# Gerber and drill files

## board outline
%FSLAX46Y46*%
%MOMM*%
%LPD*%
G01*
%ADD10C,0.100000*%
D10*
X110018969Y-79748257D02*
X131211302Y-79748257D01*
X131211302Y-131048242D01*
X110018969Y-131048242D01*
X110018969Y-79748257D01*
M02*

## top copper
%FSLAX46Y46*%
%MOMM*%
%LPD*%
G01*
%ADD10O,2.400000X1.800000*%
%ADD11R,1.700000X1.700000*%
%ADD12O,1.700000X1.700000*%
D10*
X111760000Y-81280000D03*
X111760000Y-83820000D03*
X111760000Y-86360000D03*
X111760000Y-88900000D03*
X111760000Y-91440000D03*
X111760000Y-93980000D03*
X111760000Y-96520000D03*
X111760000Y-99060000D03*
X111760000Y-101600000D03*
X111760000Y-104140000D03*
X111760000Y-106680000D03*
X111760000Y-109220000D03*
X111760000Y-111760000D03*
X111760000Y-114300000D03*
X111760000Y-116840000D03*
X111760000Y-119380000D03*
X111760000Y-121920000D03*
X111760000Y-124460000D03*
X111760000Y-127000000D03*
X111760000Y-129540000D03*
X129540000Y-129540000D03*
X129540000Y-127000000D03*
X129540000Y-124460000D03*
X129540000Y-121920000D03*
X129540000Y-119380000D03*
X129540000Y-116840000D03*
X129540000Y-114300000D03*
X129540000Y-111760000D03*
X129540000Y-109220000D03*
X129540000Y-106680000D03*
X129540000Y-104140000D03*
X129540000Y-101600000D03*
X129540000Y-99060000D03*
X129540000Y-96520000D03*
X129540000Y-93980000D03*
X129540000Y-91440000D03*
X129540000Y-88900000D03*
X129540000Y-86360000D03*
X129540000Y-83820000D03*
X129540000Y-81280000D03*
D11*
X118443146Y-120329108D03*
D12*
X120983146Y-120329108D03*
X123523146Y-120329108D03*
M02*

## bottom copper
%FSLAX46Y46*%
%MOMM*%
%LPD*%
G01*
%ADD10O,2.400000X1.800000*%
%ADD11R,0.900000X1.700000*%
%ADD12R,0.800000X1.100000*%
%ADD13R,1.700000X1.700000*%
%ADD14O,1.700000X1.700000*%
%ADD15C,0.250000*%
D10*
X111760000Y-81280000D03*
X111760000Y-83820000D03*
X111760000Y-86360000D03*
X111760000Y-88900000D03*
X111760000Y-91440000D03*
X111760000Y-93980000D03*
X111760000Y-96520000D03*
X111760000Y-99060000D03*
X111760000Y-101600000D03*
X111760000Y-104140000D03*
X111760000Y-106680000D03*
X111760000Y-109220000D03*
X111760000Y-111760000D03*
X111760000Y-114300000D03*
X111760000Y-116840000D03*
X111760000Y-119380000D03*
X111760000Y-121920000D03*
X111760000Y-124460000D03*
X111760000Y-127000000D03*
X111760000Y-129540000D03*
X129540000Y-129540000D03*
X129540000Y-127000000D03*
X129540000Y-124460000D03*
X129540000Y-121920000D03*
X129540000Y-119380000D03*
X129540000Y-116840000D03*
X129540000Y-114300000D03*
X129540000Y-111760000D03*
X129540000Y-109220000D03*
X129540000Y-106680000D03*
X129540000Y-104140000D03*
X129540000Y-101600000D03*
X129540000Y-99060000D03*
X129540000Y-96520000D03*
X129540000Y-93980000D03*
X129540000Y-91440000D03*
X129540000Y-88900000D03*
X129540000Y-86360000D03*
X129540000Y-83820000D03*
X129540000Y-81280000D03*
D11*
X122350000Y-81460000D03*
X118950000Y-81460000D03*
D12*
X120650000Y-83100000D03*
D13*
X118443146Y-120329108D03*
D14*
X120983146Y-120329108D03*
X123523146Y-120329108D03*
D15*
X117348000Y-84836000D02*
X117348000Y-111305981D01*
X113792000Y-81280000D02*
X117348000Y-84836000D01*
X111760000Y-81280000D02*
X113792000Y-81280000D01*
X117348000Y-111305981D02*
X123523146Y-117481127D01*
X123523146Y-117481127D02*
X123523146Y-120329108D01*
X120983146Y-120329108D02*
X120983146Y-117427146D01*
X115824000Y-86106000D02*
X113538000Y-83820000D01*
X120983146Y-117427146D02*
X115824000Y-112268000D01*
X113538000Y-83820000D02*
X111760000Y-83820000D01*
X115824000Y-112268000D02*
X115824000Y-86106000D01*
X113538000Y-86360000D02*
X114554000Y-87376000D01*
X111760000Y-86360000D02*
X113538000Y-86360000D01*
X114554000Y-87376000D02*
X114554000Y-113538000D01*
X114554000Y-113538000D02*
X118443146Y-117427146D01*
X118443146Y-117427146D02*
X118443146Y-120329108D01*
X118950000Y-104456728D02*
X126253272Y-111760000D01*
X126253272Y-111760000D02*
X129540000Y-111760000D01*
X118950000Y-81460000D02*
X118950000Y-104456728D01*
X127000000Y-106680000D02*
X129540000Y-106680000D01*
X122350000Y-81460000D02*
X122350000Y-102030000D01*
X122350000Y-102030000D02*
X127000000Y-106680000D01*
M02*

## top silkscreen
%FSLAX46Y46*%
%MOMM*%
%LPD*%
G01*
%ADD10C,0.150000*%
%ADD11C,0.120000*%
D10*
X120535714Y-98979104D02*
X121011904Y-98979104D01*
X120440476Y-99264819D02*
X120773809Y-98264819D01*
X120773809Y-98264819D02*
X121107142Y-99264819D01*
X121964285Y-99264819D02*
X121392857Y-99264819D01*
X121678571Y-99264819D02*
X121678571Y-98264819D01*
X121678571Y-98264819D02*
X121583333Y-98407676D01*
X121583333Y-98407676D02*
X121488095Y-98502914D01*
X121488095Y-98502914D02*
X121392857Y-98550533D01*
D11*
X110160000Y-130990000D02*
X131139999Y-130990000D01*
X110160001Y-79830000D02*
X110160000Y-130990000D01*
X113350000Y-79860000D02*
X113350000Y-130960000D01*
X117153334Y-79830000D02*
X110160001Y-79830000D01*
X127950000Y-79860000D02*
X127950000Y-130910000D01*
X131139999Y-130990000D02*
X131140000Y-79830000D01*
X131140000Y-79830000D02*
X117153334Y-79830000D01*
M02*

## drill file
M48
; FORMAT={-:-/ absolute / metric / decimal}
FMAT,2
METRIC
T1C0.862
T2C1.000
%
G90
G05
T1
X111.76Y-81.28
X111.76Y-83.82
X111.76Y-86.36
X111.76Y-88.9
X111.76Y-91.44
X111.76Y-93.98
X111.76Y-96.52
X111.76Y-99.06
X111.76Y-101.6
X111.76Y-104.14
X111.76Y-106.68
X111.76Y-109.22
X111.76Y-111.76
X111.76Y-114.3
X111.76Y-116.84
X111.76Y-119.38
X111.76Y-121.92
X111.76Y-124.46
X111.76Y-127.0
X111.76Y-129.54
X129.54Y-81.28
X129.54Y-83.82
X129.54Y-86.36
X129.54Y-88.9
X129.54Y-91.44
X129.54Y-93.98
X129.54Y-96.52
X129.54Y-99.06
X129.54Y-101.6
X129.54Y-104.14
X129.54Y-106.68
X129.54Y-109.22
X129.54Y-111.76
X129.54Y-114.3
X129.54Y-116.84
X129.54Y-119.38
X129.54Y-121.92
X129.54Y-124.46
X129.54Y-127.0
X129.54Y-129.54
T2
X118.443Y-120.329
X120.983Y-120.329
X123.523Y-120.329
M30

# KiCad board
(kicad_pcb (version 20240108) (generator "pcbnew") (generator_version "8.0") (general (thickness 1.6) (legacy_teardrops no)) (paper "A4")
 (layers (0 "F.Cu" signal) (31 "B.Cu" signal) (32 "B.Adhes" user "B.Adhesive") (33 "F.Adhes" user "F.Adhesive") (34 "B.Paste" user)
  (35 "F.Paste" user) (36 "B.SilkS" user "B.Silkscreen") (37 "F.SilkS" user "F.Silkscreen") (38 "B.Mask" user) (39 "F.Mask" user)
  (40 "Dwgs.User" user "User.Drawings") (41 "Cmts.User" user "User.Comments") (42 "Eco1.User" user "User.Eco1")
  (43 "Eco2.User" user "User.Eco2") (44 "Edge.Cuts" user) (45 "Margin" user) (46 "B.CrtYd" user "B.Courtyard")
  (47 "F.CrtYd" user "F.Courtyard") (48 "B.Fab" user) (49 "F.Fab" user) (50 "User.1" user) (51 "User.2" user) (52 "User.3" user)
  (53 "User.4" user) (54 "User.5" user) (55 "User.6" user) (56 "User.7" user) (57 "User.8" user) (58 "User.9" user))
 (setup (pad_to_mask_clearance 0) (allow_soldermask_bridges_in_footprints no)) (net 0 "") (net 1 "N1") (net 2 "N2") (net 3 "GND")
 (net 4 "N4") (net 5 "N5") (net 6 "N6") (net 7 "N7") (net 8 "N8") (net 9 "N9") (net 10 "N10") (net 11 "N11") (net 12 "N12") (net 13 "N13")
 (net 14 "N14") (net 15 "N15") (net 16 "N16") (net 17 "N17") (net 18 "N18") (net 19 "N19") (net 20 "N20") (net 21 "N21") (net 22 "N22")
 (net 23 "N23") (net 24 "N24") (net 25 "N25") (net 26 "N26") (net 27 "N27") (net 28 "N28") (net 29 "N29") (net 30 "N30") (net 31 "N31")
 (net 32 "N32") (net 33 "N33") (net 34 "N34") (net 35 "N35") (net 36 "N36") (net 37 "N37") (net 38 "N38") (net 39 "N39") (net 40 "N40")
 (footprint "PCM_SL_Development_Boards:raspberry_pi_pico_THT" (layer "F.Cu") (at 111.76 81.28)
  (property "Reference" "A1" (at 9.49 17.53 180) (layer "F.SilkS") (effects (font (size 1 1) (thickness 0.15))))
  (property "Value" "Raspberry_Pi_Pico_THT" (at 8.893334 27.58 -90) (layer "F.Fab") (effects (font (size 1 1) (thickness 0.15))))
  (fp_line (start -1.6 49.71) (end 19.379999 49.71) (stroke (width 0.12) (type solid)) (layer "F.SilkS"))
  (fp_line (start -1.599999 -1.45) (end -1.6 49.71) (stroke (width 0.12) (type solid)) (layer "F.SilkS"))
  (fp_line (start 1.59 -1.42) (end 1.59 49.68) (stroke (width 0.12) (type solid)) (layer "F.SilkS"))
  (fp_line (start 5.393334 -1.45) (end -1.599999 -1.45) (stroke (width 0.12) (type solid)) (layer "F.SilkS"))
  (fp_line (start 16.19 -1.42) (end 16.19 49.63) (stroke (width 0.12) (type solid)) (layer "F.SilkS"))
  (fp_line (start 19.379999 49.71) (end 19.38 -1.45) (stroke (width 0.12) (type solid)) (layer "F.SilkS"))
  (fp_line (start 19.38 -1.45) (end 5.393334 -1.45) (stroke (width 0.12) (type solid)) (layer "F.SilkS"))
  (pad "1" thru_hole oval (at 0 0 270) (size 1.8 2.4) (drill 0.862) (layers "*.Cu" "*.Mask") (remove_unused_layers no) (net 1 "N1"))
  (pad "2" thru_hole oval (at 0 2.54 270) (size 1.8 2.4) (drill 0.862) (layers "*.Cu" "*.Mask") (remove_unused_layers no) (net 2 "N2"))
  (pad "3" thru_hole oval (at 0 5.08 270) (size 1.8 2.4) (drill 0.862) (layers "*.Cu" "*.Mask") (remove_unused_layers no) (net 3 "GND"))
  (pad "4" thru_hole oval (at 0 7.62 270) (size 1.8 2.4) (drill 0.862) (layers "*.Cu" "*.Mask") (remove_unused_layers no) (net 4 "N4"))
  (pad "5" thru_hole oval (at 0 10.16 270) (size 1.8 2.4) (drill 0.862) (layers "*.Cu" "*.Mask") (remove_unused_layers no) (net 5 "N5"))
  (pad "6" thru_hole oval (at 0 12.7 270) (size 1.8 2.4) (drill 0.862) (layers "*.Cu" "*.Mask") (remove_unused_layers no) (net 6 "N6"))
  (pad "7" thru_hole oval (at 0 15.24 270) (size 1.8 2.4) (drill 0.862) (layers "*.Cu" "*.Mask") (remove_unused_layers no) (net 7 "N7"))
  (pad "8" thru_hole oval (at 0 17.78 270) (size 1.8 2.4) (drill 0.862) (layers "*.Cu" "*.Mask") (remove_unused_layers no) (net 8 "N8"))
  (pad "9" thru_hole oval (at 0 20.32 270) (size 1.8 2.4) (drill 0.862) (layers "*.Cu" "*.Mask") (remove_unused_layers no) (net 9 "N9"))
  (pad "10" thru_hole oval (at 0 22.86 270) (size 1.8 2.4) (drill 0.862) (layers "*.Cu" "*.Mask") (remove_unused_layers no) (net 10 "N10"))
  (pad "11" thru_hole oval (at 0 25.4 270) (size 1.8 2.4) (drill 0.862) (layers "*.Cu" "*.Mask") (remove_unused_layers no) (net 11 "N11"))
  (pad "12" thru_hole oval (at 0 27.94 270) (size 1.8 2.4) (drill 0.862) (layers "*.Cu" "*.Mask") (remove_unused_layers no) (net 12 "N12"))
  (pad "13" thru_hole oval (at 0 30.48 270) (size 1.8 2.4) (drill 0.862) (layers "*.Cu" "*.Mask") (remove_unused_layers no) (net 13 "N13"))
  (pad "14" thru_hole oval (at 0 33.02 270) (size 1.8 2.4) (drill 0.862) (layers "*.Cu" "*.Mask") (remove_unused_layers no) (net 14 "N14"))
  (pad "15" thru_hole oval (at 0 35.56 270) (size 1.8 2.4) (drill 0.862) (layers "*.Cu" "*.Mask") (remove_unused_layers no) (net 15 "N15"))
  (pad "16" thru_hole oval (at 0 38.1 270) (size 1.8 2.4) (drill 0.862) (layers "*.Cu" "*.Mask") (remove_unused_layers no) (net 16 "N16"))
  (pad "17" thru_hole oval (at 0 40.64 270) (size 1.8 2.4) (drill 0.862) (layers "*.Cu" "*.Mask") (remove_unused_layers no) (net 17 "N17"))
  (pad "18" thru_hole oval (at 0 43.18 270) (size 1.8 2.4) (drill 0.862) (layers "*.Cu" "*.Mask") (remove_unused_layers no) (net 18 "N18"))
  (pad "19" thru_hole oval (at 0 45.72 270) (size 1.8 2.4) (drill 0.862) (layers "*.Cu" "*.Mask") (remove_unused_layers no) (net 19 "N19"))
  (pad "20" thru_hole oval (at 0 48.26 270) (size 1.8 2.4) (drill 0.862) (layers "*.Cu" "*.Mask") (remove_unused_layers no) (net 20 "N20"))
  (pad "21" thru_hole oval (at 17.78 48.26 270) (size 1.8 2.4) (drill 0.862) (layers "*.Cu" "*.Mask") (remove_unused_layers no)
   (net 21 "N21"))
  (pad "22" thru_hole oval (at 17.78 45.72 270) (size 1.8 2.4) (drill 0.862) (layers "*.Cu" "*.Mask") (remove_unused_layers no)
   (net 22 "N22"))
  (pad "23" thru_hole oval (at 17.78 43.18 270) (size 1.8 2.4) (drill 0.862) (layers "*.Cu" "*.Mask") (remove_unused_layers no)
   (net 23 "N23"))
  (pad "24" thru_hole oval (at 17.78 40.64 270) (size 1.8 2.4) (drill 0.862) (layers "*.Cu" "*.Mask") (remove_unused_layers no)
   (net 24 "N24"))
  (pad "25" thru_hole oval (at 17.78 38.1 270) (size 1.8 2.4) (drill 0.862) (layers "*.Cu" "*.Mask") (remove_unused_layers no)
   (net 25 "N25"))
  (pad "26" thru_hole oval (at 17.78 35.56 270) (size 1.8 2.4) (drill 0.862) (layers "*.Cu" "*.Mask") (remove_unused_layers no)
   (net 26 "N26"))
  (pad "27" thru_hole oval (at 17.78 33.02 270) (size 1.8 2.4) (drill 0.862) (layers "*.Cu" "*.Mask") (remove_unused_layers no)
   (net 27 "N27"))
  (pad "28" thru_hole oval (at 17.78 30.48 270) (size 1.8 2.4) (drill 0.862) (layers "*.Cu" "*.Mask") (remove_unused_layers no)
   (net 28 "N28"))
  (pad "29" thru_hole oval (at 17.78 27.94 270) (size 1.8 2.4) (drill 0.862) (layers "*.Cu" "*.Mask") (remove_unused_layers no)
   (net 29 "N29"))
  (pad "30" thru_hole oval (at 17.78 25.4 270) (size 1.8 2.4) (drill 0.862) (layers "*.Cu" "*.Mask") (remove_unused_layers no)
   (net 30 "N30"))
  (pad "31" thru_hole oval (at 17.78 22.86 270) (size 1.8 2.4) (drill 0.862) (layers "*.Cu" "*.Mask") (remove_unused_layers no)
   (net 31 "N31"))
  (pad "32" thru_hole oval (at 17.78 20.32 270) (size 1.8 2.4) (drill 0.862) (layers "*.Cu" "*.Mask") (remove_unused_layers no)
   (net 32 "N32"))
  (pad "33" thru_hole oval (at 17.78 17.78 270) (size 1.8 2.4) (drill 0.862) (layers "*.Cu" "*.Mask") (remove_unused_layers no)
   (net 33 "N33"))
  (pad "34" thru_hole oval (at 17.78 15.24 270) (size 1.8 2.4) (drill 0.862) (layers "*.Cu" "*.Mask") (remove_unused_layers no)
   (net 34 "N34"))
  (pad "35" thru_hole oval (at 17.78 12.7 270) (size 1.8 2.4) (drill 0.862) (layers "*.Cu" "*.Mask") (remove_unused_layers no)
   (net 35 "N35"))
  (pad "36" thru_hole oval (at 17.78 10.16 270) (size 1.8 2.4) (drill 0.862) (layers "*.Cu" "*.Mask") (remove_unused_layers no)
   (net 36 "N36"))
  (pad "37" thru_hole oval (at 17.78 7.62 270) (size 1.8 2.4) (drill 0.862) (layers "*.Cu" "*.Mask") (remove_unused_layers no)
   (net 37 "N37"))
  (pad "38" thru_hole oval (at 17.78 5.08 270) (size 1.8 2.4) (drill 0.862) (layers "*.Cu" "*.Mask") (remove_unused_layers no)
   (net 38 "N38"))
  (pad "39" thru_hole oval (at 17.78 2.54 270) (size 1.8 2.4) (drill 0.862) (layers "*.Cu" "*.Mask") (remove_unused_layers no)
   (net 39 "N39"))
  (pad "40" thru_hole oval (at 17.78 0 270) (size 1.8 2.4) (drill 0.862) (layers "*.Cu" "*.Mask") (remove_unused_layers no) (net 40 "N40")))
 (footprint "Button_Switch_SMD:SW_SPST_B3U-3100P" (layer "B.Cu") (at 120.65 82.28 180)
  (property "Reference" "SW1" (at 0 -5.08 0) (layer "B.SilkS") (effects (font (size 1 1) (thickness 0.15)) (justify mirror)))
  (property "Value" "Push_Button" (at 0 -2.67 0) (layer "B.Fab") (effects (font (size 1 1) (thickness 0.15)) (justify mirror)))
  (pad "1" smd rect (at -1.7 0.82 180) (size 0.9 1.7) (layers "B.Cu" "B.Paste" "B.Mask") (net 30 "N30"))
  (pad "2" smd rect (at 1.7 0.82 180) (size 0.9 1.7) (layers "B.Cu" "B.Paste" "B.Mask") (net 28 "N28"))
  (pad "3" smd rect (at 0 -0.82 180) (size 0.8 1.1) (layers "B.Cu" "B.Paste" "B.Mask")))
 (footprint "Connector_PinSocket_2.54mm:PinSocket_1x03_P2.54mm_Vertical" (layer "B.Cu") (at 118.443146 120.329108 -90)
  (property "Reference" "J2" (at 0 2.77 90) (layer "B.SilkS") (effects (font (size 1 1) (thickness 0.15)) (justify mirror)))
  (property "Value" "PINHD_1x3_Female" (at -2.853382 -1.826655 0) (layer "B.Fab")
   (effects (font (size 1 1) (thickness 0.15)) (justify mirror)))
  (pad "1" thru_hole rect (at 0 0 270) (size 1.7 1.7) (drill 1) (layers "*.Cu" "*.Mask") (remove_unused_layers no) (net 3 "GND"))
  (pad "2" thru_hole oval (at 0 -2.54 270) (size 1.7 1.7) (drill 1) (layers "*.Cu" "*.Mask") (remove_unused_layers no) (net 2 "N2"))
  (pad "3" thru_hole oval (at 0 -5.08 270) (size 1.7 1.7) (drill 1) (layers "*.Cu" "*.Mask") (remove_unused_layers no) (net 1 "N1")))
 (gr_rect (start 110.018969 79.748257) (end 131.211302 131.048242) (stroke (width 0.1) (type default)) (fill none) (layer "Edge.Cuts"))
 (segment (start 117.348 84.836) (end 117.348 111.305981) (width 0.25) (layer "B.Cu") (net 1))
 (segment (start 113.792 81.28) (end 117.348 84.836) (width 0.25) (layer "B.Cu") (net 1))
 (segment (start 111.76 81.28) (end 113.792 81.28) (width 0.25) (layer "B.Cu") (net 1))
 (segment (start 117.348 111.305981) (end 123.523146 117.481127) (width 0.25) (layer "B.Cu") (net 1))
 (segment (start 123.523146 117.481127) (end 123.523146 120.329108) (width 0.25) (layer "B.Cu") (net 1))
 (segment (start 120.983146 120.329108) (end 120.983146 117.427146) (width 0.25) (layer "B.Cu") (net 2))
 (segment (start 115.824 86.106) (end 113.538 83.82) (width 0.25) (layer "B.Cu") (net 2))
 (segment (start 120.983146 117.427146) (end 115.824 112.268) (width 0.25) (layer "B.Cu") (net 2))
 (segment (start 113.538 83.82) (end 111.76 83.82) (width 0.25) (layer "B.Cu") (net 2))
 (segment (start 115.824 112.268) (end 115.824 86.106) (width 0.25) (layer "B.Cu") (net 2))
 (segment (start 113.538 86.36) (end 114.554 87.376) (width 0.25) (layer "B.Cu") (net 3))
 (segment (start 111.76 86.36) (end 113.538 86.36) (width 0.25) (layer "B.Cu") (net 3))
 (segment (start 114.554 87.376) (end 114.554 113.538) (width 0.25) (layer "B.Cu") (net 3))
 (segment (start 114.554 113.538) (end 118.443146 117.427146) (width 0.25) (layer "B.Cu") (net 3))
 (segment (start 118.443146 117.427146) (end 118.443146 120.329108) (width 0.25) (layer "B.Cu") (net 3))
 (segment (start 118.95 104.456728) (end 126.253272 111.76) (width 0.25) (layer "B.Cu") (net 28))
 (segment (start 126.253272 111.76) (end 129.54 111.76) (width 0.25) (layer "B.Cu") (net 28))
 (segment (start 118.95 81.46) (end 118.95 104.456728) (width 0.25) (layer "B.Cu") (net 28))
 (segment (start 127 106.68) (end 129.54 106.68) (width 0.25) (layer "B.Cu") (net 30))
 (segment (start 122.35 81.46) (end 122.35 102.03) (width 0.25) (layer "B.Cu") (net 30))
 (segment (start 122.35 102.03) (end 127 106.68) (width 0.25) (layer "B.Cu") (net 30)))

